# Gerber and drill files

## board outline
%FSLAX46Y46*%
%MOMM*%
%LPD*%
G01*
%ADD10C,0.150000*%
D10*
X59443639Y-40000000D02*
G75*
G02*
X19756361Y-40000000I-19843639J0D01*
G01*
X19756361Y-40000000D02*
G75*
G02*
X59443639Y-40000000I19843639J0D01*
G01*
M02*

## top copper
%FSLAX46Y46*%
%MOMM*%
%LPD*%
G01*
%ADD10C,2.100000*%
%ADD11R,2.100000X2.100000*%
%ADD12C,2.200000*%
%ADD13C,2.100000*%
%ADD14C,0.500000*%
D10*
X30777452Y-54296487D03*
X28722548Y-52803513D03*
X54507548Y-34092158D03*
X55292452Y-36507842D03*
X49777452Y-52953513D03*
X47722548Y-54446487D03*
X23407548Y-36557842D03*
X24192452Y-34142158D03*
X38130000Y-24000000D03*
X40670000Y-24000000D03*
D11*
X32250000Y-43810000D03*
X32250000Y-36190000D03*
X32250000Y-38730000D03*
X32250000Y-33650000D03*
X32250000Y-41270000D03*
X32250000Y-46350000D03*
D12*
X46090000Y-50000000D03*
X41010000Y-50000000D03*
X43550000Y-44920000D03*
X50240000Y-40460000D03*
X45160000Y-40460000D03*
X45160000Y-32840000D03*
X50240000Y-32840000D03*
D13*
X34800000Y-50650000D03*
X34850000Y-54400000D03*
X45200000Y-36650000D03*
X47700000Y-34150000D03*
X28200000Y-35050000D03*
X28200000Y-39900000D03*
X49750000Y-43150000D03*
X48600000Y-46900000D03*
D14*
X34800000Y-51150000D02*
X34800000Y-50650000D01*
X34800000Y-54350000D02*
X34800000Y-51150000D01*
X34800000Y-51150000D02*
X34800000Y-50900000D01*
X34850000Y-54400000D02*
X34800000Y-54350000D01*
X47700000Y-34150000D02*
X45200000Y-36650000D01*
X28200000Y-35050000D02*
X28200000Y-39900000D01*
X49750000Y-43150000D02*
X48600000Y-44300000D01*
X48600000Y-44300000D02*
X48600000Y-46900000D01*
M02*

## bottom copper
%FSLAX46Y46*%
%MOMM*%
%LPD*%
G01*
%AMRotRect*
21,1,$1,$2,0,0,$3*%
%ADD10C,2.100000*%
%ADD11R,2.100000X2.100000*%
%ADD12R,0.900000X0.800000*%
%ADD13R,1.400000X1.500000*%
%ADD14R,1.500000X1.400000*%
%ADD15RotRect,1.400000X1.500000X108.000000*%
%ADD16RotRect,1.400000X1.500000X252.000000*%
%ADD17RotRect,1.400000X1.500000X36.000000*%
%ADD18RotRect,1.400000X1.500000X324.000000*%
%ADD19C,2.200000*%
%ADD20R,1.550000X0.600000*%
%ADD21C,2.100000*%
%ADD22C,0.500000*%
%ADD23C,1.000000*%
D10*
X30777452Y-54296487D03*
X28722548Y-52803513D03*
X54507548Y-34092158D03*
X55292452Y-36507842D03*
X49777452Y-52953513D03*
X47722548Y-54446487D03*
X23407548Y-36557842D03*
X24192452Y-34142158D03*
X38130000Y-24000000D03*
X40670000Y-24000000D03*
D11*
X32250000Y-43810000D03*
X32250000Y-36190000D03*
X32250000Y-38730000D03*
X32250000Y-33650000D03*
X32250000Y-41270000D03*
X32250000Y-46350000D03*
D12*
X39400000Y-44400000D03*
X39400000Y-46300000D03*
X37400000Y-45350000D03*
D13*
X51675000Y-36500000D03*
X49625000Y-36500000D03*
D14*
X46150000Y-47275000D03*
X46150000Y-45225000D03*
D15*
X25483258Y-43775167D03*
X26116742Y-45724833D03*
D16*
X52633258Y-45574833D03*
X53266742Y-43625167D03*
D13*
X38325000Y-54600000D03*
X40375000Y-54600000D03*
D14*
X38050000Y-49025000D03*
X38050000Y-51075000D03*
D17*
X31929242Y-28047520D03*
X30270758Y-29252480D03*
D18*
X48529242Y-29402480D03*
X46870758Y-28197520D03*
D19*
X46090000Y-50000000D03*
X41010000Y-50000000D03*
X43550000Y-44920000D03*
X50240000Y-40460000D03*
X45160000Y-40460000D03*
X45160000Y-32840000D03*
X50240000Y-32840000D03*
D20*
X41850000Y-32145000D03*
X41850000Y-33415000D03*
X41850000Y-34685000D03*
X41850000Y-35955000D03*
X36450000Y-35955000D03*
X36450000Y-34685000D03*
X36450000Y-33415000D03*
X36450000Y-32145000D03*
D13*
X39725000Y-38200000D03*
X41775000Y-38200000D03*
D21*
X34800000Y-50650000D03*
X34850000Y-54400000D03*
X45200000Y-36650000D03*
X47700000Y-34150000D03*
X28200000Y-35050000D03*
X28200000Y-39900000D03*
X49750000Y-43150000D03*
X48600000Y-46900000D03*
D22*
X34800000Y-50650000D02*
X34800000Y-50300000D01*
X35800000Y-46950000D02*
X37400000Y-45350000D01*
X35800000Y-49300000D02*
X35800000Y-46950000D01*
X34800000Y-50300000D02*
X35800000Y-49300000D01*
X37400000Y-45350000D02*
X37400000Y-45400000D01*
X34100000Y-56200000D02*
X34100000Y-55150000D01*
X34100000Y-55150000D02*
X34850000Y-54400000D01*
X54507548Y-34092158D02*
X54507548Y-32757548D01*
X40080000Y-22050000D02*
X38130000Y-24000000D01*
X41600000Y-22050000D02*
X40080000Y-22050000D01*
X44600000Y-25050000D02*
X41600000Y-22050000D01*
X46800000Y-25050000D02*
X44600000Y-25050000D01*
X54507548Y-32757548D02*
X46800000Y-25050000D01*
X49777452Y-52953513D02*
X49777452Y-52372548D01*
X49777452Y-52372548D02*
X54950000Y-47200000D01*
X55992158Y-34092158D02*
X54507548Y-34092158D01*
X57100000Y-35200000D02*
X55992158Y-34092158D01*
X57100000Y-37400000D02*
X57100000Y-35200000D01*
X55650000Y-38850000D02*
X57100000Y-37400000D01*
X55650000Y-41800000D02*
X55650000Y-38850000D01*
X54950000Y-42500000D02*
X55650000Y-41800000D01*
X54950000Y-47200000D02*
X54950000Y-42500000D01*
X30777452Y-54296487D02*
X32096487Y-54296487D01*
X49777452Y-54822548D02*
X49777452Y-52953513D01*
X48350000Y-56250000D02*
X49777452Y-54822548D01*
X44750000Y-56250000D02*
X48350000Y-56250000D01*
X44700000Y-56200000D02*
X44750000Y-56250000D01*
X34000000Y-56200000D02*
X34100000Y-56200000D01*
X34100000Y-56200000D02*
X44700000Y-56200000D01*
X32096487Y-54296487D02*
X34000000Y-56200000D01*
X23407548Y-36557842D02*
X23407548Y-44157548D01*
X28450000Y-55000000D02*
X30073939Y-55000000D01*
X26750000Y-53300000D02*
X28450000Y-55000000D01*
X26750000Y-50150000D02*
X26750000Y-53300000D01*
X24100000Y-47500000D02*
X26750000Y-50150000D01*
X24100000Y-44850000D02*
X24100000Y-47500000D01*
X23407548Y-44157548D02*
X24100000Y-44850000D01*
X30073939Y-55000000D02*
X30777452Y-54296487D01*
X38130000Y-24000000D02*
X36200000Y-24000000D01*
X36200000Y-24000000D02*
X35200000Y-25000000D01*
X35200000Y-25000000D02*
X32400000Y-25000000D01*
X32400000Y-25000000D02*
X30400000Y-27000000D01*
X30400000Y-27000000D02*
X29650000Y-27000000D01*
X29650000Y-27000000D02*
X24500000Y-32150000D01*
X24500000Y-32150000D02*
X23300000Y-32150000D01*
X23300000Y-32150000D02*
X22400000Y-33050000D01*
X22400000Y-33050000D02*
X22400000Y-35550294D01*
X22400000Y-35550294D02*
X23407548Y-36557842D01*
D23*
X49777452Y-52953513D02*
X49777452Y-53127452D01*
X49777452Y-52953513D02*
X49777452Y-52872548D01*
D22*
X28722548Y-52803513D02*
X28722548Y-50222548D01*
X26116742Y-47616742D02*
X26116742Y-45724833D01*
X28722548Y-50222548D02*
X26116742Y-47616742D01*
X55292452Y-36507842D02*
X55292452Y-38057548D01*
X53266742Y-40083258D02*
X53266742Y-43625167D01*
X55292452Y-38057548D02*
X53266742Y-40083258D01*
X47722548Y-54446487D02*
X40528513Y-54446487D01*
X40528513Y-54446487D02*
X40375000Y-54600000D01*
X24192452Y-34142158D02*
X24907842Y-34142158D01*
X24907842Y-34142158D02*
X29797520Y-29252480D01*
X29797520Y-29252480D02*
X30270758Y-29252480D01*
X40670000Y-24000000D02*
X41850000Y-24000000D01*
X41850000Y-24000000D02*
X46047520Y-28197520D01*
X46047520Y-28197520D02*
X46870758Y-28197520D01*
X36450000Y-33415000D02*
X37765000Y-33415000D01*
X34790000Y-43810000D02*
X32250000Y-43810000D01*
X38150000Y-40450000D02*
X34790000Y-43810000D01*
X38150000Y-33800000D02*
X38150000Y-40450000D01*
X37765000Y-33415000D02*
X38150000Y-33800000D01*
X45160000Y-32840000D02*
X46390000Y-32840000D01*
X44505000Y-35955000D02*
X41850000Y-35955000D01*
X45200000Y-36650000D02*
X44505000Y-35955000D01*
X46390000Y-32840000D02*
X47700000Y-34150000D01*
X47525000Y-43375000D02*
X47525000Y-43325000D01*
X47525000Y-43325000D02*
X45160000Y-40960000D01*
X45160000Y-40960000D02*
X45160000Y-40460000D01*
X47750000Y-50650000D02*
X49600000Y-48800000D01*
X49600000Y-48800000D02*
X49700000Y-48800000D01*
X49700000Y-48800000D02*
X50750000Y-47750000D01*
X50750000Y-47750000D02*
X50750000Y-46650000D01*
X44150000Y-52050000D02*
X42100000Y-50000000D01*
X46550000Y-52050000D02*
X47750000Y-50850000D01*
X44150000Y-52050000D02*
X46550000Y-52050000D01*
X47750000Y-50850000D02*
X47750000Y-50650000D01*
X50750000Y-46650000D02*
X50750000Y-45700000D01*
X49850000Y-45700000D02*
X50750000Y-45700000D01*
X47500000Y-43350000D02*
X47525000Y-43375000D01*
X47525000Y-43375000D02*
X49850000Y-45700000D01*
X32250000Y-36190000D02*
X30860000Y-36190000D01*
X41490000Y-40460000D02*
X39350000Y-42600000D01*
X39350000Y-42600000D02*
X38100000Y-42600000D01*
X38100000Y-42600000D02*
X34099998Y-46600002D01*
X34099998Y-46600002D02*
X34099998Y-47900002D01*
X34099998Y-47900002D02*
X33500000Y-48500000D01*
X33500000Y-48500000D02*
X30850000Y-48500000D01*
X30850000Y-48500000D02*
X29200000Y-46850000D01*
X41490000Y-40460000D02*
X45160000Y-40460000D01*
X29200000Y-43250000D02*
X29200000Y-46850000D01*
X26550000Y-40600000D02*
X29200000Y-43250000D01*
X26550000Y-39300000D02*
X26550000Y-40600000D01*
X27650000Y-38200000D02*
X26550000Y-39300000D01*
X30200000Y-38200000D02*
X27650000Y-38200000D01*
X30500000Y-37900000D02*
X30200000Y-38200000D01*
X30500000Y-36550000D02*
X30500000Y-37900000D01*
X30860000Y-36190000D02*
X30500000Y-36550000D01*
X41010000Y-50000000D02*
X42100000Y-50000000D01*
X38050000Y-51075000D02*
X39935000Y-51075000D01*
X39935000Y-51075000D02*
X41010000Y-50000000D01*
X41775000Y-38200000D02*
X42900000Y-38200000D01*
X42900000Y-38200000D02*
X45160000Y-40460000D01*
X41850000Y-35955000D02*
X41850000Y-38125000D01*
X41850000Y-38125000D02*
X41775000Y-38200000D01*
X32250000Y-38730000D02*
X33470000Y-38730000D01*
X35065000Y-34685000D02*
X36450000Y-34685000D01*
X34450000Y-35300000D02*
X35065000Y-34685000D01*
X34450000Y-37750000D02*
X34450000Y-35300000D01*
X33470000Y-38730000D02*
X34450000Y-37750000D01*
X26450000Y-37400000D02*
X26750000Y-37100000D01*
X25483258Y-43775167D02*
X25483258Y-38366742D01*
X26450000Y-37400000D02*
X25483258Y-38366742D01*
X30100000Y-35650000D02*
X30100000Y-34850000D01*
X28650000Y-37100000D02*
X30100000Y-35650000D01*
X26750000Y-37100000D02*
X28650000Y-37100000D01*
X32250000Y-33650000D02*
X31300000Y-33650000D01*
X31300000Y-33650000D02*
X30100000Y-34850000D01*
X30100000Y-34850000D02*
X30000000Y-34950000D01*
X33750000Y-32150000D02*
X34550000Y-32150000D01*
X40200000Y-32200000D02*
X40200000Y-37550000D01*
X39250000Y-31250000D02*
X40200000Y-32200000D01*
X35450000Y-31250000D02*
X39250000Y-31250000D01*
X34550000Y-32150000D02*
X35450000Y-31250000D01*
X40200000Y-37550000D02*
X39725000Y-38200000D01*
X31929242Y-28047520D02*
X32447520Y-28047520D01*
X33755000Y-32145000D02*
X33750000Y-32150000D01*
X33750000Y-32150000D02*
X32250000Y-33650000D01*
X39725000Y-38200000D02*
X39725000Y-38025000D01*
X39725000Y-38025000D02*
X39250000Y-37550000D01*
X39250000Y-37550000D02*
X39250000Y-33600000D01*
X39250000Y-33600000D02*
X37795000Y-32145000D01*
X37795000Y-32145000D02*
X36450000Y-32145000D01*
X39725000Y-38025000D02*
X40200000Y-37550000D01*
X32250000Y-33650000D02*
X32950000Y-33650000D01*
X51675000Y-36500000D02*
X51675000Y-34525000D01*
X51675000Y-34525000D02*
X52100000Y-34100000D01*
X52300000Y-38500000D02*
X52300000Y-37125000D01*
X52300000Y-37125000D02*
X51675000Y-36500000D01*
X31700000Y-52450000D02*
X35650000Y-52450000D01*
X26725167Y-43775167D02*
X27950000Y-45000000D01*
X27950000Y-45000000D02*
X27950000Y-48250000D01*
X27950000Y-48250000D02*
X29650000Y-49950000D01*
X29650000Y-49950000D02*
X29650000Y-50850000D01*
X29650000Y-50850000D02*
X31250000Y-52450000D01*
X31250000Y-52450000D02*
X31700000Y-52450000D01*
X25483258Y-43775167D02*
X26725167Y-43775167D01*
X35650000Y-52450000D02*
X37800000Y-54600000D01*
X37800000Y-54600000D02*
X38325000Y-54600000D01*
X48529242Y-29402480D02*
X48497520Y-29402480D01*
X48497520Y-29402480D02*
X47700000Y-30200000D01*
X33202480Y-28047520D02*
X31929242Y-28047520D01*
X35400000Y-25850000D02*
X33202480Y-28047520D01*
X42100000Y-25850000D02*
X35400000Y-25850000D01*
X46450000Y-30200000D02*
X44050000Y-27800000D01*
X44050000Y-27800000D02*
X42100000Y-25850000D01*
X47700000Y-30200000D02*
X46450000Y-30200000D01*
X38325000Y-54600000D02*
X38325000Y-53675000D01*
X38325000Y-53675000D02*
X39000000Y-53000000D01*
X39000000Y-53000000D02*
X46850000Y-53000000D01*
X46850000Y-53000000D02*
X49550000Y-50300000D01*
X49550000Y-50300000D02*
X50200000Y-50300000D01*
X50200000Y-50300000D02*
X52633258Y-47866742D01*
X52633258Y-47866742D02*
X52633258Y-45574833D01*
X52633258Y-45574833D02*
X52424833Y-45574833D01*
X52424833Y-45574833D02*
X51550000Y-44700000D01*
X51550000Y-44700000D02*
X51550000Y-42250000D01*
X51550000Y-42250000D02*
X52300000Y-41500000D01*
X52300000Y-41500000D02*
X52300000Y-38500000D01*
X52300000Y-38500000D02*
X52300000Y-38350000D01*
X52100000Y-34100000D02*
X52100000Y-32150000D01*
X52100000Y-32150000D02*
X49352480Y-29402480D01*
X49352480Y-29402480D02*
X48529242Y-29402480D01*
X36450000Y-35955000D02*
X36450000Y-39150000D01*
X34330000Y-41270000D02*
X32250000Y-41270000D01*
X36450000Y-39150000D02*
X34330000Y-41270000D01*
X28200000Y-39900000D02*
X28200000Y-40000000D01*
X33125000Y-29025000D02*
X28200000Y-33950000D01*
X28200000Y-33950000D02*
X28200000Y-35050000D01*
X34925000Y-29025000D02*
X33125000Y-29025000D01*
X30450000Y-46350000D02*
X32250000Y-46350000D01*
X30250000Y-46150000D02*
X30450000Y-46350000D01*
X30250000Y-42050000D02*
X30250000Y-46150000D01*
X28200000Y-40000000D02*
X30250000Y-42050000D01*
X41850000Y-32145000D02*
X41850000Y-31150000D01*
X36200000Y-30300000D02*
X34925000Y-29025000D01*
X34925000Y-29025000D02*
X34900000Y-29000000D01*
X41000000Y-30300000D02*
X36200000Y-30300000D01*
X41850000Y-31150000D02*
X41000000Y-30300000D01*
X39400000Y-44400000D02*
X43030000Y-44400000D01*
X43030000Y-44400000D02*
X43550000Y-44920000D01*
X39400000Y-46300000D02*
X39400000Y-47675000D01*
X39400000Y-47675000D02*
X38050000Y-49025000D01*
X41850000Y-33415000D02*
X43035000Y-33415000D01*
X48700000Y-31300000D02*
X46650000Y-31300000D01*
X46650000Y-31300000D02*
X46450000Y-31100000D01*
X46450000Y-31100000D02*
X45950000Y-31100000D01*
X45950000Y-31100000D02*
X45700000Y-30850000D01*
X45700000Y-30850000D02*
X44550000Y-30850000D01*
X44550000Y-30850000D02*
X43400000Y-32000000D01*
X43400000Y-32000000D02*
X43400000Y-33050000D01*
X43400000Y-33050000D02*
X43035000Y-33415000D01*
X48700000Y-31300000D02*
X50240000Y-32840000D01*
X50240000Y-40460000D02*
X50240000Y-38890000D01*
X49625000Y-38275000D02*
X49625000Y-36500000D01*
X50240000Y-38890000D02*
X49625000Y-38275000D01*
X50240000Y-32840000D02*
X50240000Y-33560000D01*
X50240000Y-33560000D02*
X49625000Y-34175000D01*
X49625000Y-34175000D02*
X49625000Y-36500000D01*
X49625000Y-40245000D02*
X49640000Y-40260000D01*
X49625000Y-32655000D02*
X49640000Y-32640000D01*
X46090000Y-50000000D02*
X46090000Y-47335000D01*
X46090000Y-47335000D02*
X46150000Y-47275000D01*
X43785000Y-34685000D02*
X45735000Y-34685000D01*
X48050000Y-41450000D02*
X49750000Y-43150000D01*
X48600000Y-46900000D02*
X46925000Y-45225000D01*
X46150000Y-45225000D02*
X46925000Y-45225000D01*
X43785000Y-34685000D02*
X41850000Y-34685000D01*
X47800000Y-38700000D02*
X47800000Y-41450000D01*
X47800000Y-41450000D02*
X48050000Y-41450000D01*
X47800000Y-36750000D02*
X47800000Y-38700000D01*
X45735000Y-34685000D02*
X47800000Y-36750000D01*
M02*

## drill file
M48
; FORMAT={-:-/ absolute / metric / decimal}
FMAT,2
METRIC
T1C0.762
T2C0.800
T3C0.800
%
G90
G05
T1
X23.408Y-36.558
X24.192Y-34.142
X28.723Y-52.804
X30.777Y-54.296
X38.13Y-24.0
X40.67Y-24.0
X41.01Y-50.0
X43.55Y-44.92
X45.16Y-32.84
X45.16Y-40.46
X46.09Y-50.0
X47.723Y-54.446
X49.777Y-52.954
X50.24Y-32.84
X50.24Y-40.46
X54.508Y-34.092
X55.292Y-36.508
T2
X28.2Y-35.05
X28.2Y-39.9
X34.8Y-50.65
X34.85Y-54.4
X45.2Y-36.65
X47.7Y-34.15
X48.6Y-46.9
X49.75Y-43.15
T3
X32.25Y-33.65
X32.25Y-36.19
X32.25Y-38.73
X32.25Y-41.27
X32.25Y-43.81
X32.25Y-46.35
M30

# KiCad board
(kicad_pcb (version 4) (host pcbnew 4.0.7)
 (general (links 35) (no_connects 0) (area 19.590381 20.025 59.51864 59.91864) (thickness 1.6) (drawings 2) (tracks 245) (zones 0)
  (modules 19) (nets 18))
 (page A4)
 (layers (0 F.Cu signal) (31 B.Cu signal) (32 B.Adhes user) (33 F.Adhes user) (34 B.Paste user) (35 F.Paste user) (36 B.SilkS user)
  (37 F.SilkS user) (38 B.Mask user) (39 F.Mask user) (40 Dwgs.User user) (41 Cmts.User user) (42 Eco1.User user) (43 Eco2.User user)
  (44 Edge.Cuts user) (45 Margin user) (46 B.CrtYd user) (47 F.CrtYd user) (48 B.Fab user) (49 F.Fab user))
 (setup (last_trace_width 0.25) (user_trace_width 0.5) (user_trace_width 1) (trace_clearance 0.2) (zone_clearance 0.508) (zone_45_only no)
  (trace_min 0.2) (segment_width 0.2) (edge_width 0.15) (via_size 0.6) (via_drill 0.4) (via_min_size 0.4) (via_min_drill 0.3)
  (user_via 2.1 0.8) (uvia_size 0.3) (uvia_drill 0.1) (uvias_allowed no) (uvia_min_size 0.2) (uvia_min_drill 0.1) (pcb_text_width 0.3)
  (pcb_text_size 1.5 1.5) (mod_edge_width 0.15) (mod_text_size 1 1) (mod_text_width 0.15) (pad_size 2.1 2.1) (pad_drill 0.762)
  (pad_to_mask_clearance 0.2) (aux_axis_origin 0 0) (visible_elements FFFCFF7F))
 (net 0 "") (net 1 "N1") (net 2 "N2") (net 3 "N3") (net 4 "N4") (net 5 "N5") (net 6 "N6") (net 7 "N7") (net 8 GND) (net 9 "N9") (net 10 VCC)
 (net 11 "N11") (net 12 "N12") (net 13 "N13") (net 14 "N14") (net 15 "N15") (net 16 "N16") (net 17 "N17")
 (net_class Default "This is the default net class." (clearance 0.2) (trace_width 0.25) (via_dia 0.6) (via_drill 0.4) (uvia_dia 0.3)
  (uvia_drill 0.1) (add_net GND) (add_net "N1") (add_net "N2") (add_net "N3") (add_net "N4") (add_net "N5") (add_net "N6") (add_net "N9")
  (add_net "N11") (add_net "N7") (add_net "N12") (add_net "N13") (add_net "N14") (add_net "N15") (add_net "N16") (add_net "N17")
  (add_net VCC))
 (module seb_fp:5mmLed (layer F.Cu) (at 29.75 53.55 144)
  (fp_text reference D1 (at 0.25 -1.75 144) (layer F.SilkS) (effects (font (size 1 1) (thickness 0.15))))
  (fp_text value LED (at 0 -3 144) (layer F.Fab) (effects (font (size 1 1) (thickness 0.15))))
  (pad 1 thru_hole circle (at -1.27 0 144) (size 2.1 2.1) (drill 0.762) (layers *.Cu *.Mask) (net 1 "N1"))
  (pad 2 thru_hole circle (at 1.27 0 144) (size 2.1 2.1) (drill 0.762) (layers *.Cu *.Mask) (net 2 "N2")))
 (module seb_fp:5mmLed (layer F.Cu) (at 54.9 35.3 288)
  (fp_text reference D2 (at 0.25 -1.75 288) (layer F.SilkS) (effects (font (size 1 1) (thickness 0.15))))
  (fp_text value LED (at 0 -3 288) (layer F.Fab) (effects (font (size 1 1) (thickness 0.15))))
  (pad 1 thru_hole circle (at -1.27 0 288) (size 2.1 2.1) (drill 0.762) (layers *.Cu *.Mask) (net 1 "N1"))
  (pad 2 thru_hole circle (at 1.27 0 288) (size 2.1 2.1) (drill 0.762) (layers *.Cu *.Mask) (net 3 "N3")))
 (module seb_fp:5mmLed (layer F.Cu) (at 48.75 53.7 216)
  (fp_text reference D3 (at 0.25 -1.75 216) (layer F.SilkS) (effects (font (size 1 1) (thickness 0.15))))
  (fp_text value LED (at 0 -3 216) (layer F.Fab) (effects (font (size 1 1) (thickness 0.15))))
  (pad 1 thru_hole circle (at -1.27 0 216) (size 2.1 2.1) (drill 0.762) (layers *.Cu *.Mask) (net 1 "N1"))
  (pad 2 thru_hole circle (at 1.27 0 216) (size 2.1 2.1) (drill 0.762) (layers *.Cu *.Mask) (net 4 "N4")))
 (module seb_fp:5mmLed (layer F.Cu) (at 23.8 35.35 72)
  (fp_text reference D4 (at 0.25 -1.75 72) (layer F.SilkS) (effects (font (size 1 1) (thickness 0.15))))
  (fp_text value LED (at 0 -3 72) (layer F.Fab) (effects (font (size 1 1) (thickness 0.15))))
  (pad 1 thru_hole circle (at -1.27 0 144) (size 2.1 2.1) (drill 0.762) (layers *.Cu *.Mask) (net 1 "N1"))
  (pad 2 thru_hole circle (at 1.27 0 144) (size 2.1 2.1) (drill 0.762) (layers *.Cu *.Mask) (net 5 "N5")))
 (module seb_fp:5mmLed (layer F.Cu) (at 39.4 24)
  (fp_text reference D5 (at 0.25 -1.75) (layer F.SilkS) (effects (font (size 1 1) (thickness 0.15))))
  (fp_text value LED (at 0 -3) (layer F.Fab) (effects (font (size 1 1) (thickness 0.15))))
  (pad 1 thru_hole circle (at -1.27 0) (size 2.1 2.1) (drill 0.762) (layers *.Cu *.Mask) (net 1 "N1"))
  (pad 2 thru_hole circle (at 1.27 0) (size 2.1 2.1) (drill 0.762) (layers *.Cu *.Mask) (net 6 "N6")))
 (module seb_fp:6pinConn (layer F.Cu) (at 32.25 40)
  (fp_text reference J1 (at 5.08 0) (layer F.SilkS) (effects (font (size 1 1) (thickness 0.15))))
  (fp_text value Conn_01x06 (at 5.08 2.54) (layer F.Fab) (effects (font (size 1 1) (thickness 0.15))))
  (pad 5 thru_hole rect (at 0 3.81) (size 2.1 2.1) (drill 0.8) (layers *.Cu *.Mask) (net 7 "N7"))
  (pad 2 thru_hole rect (at 0 -3.81) (size 2.1 2.1) (drill 0.8) (layers *.Cu *.Mask) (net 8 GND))
  (pad 3 thru_hole rect (at 0 -1.27) (size 2.1 2.1) (drill 0.8) (layers *.Cu *.Mask) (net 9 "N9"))
  (pad 1 thru_hole rect (at 0 -6.35) (size 2.1 2.1) (drill 0.8) (layers *.Cu *.Mask) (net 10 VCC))
  (pad 4 thru_hole rect (at 0 1.27) (size 2.1 2.1) (drill 0.8) (layers *.Cu *.Mask) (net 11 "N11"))
  (pad 6 thru_hole rect (at 0 6.35) (size 2.1 2.1) (drill 0.8) (layers *.Cu *.Mask) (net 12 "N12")))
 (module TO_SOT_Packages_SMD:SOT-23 (layer B.Cu) (at 38.4 45.35 180)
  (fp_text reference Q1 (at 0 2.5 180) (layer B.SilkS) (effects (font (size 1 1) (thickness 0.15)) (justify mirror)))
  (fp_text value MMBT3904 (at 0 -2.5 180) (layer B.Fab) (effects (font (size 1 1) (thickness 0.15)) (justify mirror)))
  (pad 1 smd rect (at -1 0.95 180) (size 0.9 0.8) (layers B.Cu B.Paste B.Mask) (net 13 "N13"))
  (pad 2 smd rect (at -1 -0.95 180) (size 0.9 0.8) (layers B.Cu B.Paste B.Mask) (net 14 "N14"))
  (pad 3 smd rect (at 1 0 180) (size 0.9 0.8) (layers B.Cu B.Paste B.Mask) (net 1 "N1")))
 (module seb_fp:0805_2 (layer B.Cu) (at 50.65 36.5)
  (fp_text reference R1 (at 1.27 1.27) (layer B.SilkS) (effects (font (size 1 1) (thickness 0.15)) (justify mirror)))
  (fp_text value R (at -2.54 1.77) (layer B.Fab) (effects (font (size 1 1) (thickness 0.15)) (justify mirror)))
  (pad 1 smd rect (at 1.025 0) (size 1.4 1.5) (layers B.Cu B.Paste B.Mask) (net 10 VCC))
  (pad 2 smd rect (at -1.025 0) (size 1.4 1.5) (layers B.Cu B.Paste B.Mask) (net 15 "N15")))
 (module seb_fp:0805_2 (layer B.Cu) (at 46.15 46.25 270)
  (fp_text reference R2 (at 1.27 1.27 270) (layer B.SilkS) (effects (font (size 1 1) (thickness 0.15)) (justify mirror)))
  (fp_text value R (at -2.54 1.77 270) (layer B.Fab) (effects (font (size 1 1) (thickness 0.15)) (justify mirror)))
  (pad 1 smd rect (at 1.025 0 270) (size 1.4 1.5) (layers B.Cu B.Paste B.Mask) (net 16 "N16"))
  (pad 2 smd rect (at -1.025 0 270) (size 1.4 1.5) (layers B.Cu B.Paste B.Mask) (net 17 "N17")))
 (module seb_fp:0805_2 (layer B.Cu) (at 25.8 44.75 108)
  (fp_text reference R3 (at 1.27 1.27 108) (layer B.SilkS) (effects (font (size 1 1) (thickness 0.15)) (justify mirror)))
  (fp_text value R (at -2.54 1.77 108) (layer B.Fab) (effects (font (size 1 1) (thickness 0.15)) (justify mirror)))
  (pad 1 smd rect (at 1.025 0 108) (size 1.4 1.5) (layers B.Cu B.Paste B.Mask) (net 10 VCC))
  (pad 2 smd rect (at -1.025 0 108) (size 1.4 1.5) (layers B.Cu B.Paste B.Mask) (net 2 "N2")))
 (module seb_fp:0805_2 (layer B.Cu) (at 52.95 44.6 252)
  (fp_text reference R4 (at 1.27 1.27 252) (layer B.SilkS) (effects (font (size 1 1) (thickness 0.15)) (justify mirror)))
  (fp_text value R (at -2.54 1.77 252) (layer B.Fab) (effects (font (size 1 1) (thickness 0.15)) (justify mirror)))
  (pad 1 smd rect (at 1.025 0 252) (size 1.4 1.5) (layers B.Cu B.Paste B.Mask) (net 10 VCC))
  (pad 2 smd rect (at -1.025 0 252) (size 1.4 1.5) (layers B.Cu B.Paste B.Mask) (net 3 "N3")))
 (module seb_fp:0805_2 (layer B.Cu) (at 39.35 54.6 180)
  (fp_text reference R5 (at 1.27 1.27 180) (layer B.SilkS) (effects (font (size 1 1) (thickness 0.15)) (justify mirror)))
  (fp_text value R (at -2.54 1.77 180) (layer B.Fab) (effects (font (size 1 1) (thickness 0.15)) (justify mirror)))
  (pad 1 smd rect (at 1.025 0 180) (size 1.4 1.5) (layers B.Cu B.Paste B.Mask) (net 10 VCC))
  (pad 2 smd rect (at -1.025 0 180) (size 1.4 1.5) (layers B.Cu B.Paste B.Mask) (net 4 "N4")))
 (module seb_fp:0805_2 (layer B.Cu) (at 38.05 50.05 90)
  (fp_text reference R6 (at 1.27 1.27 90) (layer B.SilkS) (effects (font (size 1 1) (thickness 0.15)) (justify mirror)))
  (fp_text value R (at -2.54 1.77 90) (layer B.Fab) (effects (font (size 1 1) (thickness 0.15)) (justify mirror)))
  (pad 1 smd rect (at 1.025 0 90) (size 1.4 1.5) (layers B.Cu B.Paste B.Mask) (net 14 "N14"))
  (pad 2 smd rect (at -1.025 0 90) (size 1.4 1.5) (layers B.Cu B.Paste B.Mask) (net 8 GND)))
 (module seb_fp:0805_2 (layer B.Cu) (at 31.1 28.65 36)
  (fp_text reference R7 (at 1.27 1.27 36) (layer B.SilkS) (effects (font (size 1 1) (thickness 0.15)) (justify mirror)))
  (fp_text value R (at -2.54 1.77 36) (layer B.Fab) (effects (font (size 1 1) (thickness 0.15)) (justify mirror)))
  (pad 1 smd rect (at 1.025 0 36) (size 1.4 1.5) (layers B.Cu B.Paste B.Mask) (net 10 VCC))
  (pad 2 smd rect (at -1.025 0 36) (size 1.4 1.5) (layers B.Cu B.Paste B.Mask) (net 5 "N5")))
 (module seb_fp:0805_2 (layer B.Cu) (at 47.7 28.8 324)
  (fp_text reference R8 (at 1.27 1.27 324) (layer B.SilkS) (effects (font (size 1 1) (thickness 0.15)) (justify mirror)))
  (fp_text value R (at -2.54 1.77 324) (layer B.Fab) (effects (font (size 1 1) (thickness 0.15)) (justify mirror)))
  (pad 1 smd rect (at 1.025 0 324) (size 1.4 1.5) (layers B.Cu B.Paste B.Mask) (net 10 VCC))
  (pad 2 smd rect (at -1.025 0 324) (size 1.4 1.5) (layers B.Cu B.Paste B.Mask) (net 6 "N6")))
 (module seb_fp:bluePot (layer F.Cu) (at 43.55 50 180)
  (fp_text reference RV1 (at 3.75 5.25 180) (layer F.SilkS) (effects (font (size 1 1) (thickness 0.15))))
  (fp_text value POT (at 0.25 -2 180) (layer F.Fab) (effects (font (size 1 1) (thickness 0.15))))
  (pad 1 thru_hole circle (at -2.54 0 180) (size 2.2 2.2) (drill 0.762) (layers *.Cu *.Mask) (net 16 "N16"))
  (pad 3 thru_hole circle (at 2.54 0 180) (size 2.2 2.2) (drill 0.762) (layers *.Cu *.Mask) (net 8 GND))
  (pad 2 thru_hole circle (at 0 5.08 180) (size 2.2 2.2) (drill 0.762) (layers *.Cu *.Mask) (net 13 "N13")))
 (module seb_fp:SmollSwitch (layer F.Cu) (at 47.7 36.65 90)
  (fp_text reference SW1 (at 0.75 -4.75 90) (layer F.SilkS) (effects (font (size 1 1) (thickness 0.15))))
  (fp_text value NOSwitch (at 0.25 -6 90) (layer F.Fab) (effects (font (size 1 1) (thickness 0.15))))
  (pad 1 thru_hole circle (at -3.81 2.54 90) (size 2.2 2.2) (drill 0.762) (layers *.Cu *.Mask) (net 15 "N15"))
  (pad 2 thru_hole circle (at -3.81 -2.54 90) (size 2.2 2.2) (drill 0.762) (layers *.Cu *.Mask) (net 8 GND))
  (pad 2 thru_hole circle (at 3.81 -2.54 90) (size 2.2 2.2) (drill 0.762) (layers *.Cu *.Mask) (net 8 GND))
  (pad 1 thru_hole circle (at 3.81 2.54 90) (size 2.2 2.2) (drill 0.762) (layers *.Cu *.Mask) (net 15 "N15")))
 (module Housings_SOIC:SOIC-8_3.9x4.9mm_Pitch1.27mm (layer B.Cu) (at 39.15 34.05 180)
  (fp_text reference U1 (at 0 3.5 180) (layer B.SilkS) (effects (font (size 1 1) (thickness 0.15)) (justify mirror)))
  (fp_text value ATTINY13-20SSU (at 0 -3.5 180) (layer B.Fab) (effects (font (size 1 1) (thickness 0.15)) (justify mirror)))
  (pad 1 smd rect (at -2.7 1.905 180) (size 1.55 0.6) (layers B.Cu B.Paste B.Mask) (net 12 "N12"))
  (pad 2 smd rect (at -2.7 0.635 180) (size 1.55 0.6) (layers B.Cu B.Paste B.Mask) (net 15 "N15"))
  (pad 3 smd rect (at -2.7 -0.635 180) (size 1.55 0.6) (layers B.Cu B.Paste B.Mask) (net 17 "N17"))
  (pad 4 smd rect (at -2.7 -1.905 180) (size 1.55 0.6) (layers B.Cu B.Paste B.Mask) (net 8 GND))
  (pad 5 smd rect (at 2.7 -1.905 180) (size 1.55 0.6) (layers B.Cu B.Paste B.Mask) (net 11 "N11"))
  (pad 6 smd rect (at 2.7 -0.635 180) (size 1.55 0.6) (layers B.Cu B.Paste B.Mask) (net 9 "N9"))
  (pad 7 smd rect (at 2.7 0.635 180) (size 1.55 0.6) (layers B.Cu B.Paste B.Mask) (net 7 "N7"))
  (pad 8 smd rect (at 2.7 1.905 180) (size 1.55 0.6) (layers B.Cu B.Paste B.Mask) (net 10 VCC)))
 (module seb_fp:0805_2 (layer B.Cu) (at 40.75 38.2 180)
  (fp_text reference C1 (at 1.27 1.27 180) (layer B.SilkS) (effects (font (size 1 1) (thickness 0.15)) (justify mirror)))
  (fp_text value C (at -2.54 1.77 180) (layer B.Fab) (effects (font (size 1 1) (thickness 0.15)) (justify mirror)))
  (pad 1 smd rect (at 1.025 0 180) (size 1.4 1.5) (layers B.Cu B.Paste B.Mask) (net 10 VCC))
  (pad 2 smd rect (at -1.025 0 180) (size 1.4 1.5) (layers B.Cu B.Paste B.Mask) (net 8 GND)))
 (gr_circle (center 39.6 40) (end 56.5 50.4) (layer Edge.Cuts) (width 0.15))
 (segment (start 34.8 50.65) (end 34.8 50.3) (width 0.5) (layer B.Cu) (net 1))
 (via (at 34.8 50.65) (size 2.1) (drill 0.8) (layers F.Cu B.Cu) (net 1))
 (segment (start 34.8 51.15) (end 34.8 50.65) (width 0.5) (layer F.Cu) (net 1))
 (segment (start 35.8 46.95) (end 37.4 45.35) (width 0.5) (layer B.Cu) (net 1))
 (segment (start 35.8 49.3) (end 35.8 46.95) (width 0.5) (layer B.Cu) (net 1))
 (segment (start 34.8 50.3) (end 35.8 49.3) (width 0.5) (layer B.Cu) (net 1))
 (segment (start 37.4 45.35) (end 37.4 45.4) (width 0.5) (layer B.Cu) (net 1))
 (segment (start 34.1 56.2) (end 34.1 55.15) (width 0.5) (layer B.Cu) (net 1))
 (segment (start 34.8 54.35) (end 34.8 51.15) (width 0.5) (layer F.Cu) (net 1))
 (segment (start 34.8 51.15) (end 34.8 50.9) (width 0.5) (layer F.Cu) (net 1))
 (segment (start 34.85 54.4) (end 34.8 54.35) (width 0.5) (layer F.Cu) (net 1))
 (via (at 34.85 54.4) (size 2.1) (drill 0.8) (layers F.Cu B.Cu) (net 1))
 (segment (start 34.1 55.15) (end 34.85 54.4) (width 0.5) (layer B.Cu) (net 1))
 (segment (start 54.507548 34.092158) (end 54.507548 32.757548) (width 0.5) (layer B.Cu) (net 1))
 (segment (start 40.08 22.05) (end 38.13 24) (width 0.5) (layer B.Cu) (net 1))
 (segment (start 41.6 22.05) (end 40.08 22.05) (width 0.5) (layer B.Cu) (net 1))
 (segment (start 44.6 25.05) (end 41.6 22.05) (width 0.5) (layer B.Cu) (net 1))
 (segment (start 46.8 25.05) (end 44.6 25.05) (width 0.5) (layer B.Cu) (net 1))
 (segment (start 54.507548 32.757548) (end 46.8 25.05) (width 0.5) (layer B.Cu) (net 1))
 (segment (start 49.777452 52.953513) (end 49.777452 52.372548) (width 0.5) (layer B.Cu) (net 1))
 (segment (start 49.777452 52.372548) (end 54.95 47.2) (width 0.5) (layer B.Cu) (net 1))
 (segment (start 55.992158 34.092158) (end 54.507548 34.092158) (width 0.5) (layer B.Cu) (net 1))
 (segment (start 57.1 35.2) (end 55.992158 34.092158) (width 0.5) (layer B.Cu) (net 1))
 (segment (start 57.1 37.4) (end 57.1 35.2) (width 0.5) (layer B.Cu) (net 1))
 (segment (start 55.65 38.85) (end 57.1 37.4) (width 0.5) (layer B.Cu) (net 1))
 (segment (start 55.65 41.8) (end 55.65 38.85) (width 0.5) (layer B.Cu) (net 1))
 (segment (start 54.95 42.5) (end 55.65 41.8) (width 0.5) (layer B.Cu) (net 1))
 (segment (start 54.95 47.2) (end 54.95 42.5) (width 0.5) (layer B.Cu) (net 1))
 (segment (start 30.777452 54.296487) (end 32.096487 54.296487) (width 0.5) (layer B.Cu) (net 1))
 (segment (start 49.777452 54.822548) (end 49.777452 52.953513) (width 0.5) (layer B.Cu) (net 1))
 (segment (start 48.35 56.25) (end 49.777452 54.822548) (width 0.5) (layer B.Cu) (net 1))
 (segment (start 44.75 56.25) (end 48.35 56.25) (width 0.5) (layer B.Cu) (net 1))
 (segment (start 44.7 56.2) (end 44.75 56.25) (width 0.5) (layer B.Cu) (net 1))
 (segment (start 34 56.2) (end 34.1 56.2) (width 0.5) (layer B.Cu) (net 1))
 (segment (start 34.1 56.2) (end 44.7 56.2) (width 0.5) (layer B.Cu) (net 1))
 (segment (start 32.096487 54.296487) (end 34 56.2) (width 0.5) (layer B.Cu) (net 1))
 (segment (start 23.407548 36.557842) (end 23.407548 44.157548) (width 0.5) (layer B.Cu) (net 1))
 (segment (start 28.45 55) (end 30.073939 55) (width 0.5) (layer B.Cu) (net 1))
 (segment (start 26.75 53.3) (end 28.45 55) (width 0.5) (layer B.Cu) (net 1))
 (segment (start 26.75 50.15) (end 26.75 53.3) (width 0.5) (layer B.Cu) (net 1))
 (segment (start 24.1 47.5) (end 26.75 50.15) (width 0.5) (layer B.Cu) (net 1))
 (segment (start 24.1 44.85) (end 24.1 47.5) (width 0.5) (layer B.Cu) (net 1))
 (segment (start 23.407548 44.157548) (end 24.1 44.85) (width 0.5) (layer B.Cu) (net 1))
 (segment (start 30.073939 55) (end 30.777452 54.296487) (width 0.5) (layer B.Cu) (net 1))
 (segment (start 38.13 24) (end 36.2 24) (width 0.5) (layer B.Cu) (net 1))
 (segment (start 36.2 24) (end 35.2 25) (width 0.5) (layer B.Cu) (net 1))
 (segment (start 35.2 25) (end 32.4 25) (width 0.5) (layer B.Cu) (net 1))
 (segment (start 32.4 25) (end 30.4 27) (width 0.5) (layer B.Cu) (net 1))
 (segment (start 30.4 27) (end 29.65 27) (width 0.5) (layer B.Cu) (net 1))
 (segment (start 29.65 27) (end 24.5 32.15) (width 0.5) (layer B.Cu) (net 1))
 (segment (start 24.5 32.15) (end 23.3 32.15) (width 0.5) (layer B.Cu) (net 1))
 (segment (start 23.3 32.15) (end 22.4 33.05) (width 0.5) (layer B.Cu) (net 1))
 (segment (start 22.4 33.05) (end 22.4 35.550294) (width 0.5) (layer B.Cu) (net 1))
 (segment (start 22.4 35.550294) (end 23.407548 36.557842) (width 0.5) (layer B.Cu) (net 1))
 (segment (start 49.777452 52.953513) (end 49.777452 53.127452) (width 1) (layer B.Cu) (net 1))
 (segment (start 49.777452 52.953513) (end 49.777452 52.872548) (width 1) (layer B.Cu) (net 1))
 (segment (start 28.722548 52.803513) (end 28.722548 50.222548) (width 0.5) (layer B.Cu) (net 2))
 (segment (start 26.116742 47.616742) (end 26.116742 45.724833) (width 0.5) (layer B.Cu) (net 2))
 (segment (start 28.722548 50.222548) (end 26.116742 47.616742) (width 0.5) (layer B.Cu) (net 2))
 (segment (start 55.292452 36.507842) (end 55.292452 38.057548) (width 0.5) (layer B.Cu) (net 3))
 (segment (start 53.266742 40.083258) (end 53.266742 43.625167) (width 0.5) (layer B.Cu) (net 3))
 (segment (start 55.292452 38.057548) (end 53.266742 40.083258) (width 0.5) (layer B.Cu) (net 3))
 (segment (start 47.722548 54.446487) (end 40.528513 54.446487) (width 0.5) (layer B.Cu) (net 4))
 (segment (start 40.528513 54.446487) (end 40.375 54.6) (width 0.5) (layer B.Cu) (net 4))
 (segment (start 24.192452 34.142158) (end 24.907842 34.142158) (width 0.5) (layer B.Cu) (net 5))
 (segment (start 24.907842 34.142158) (end 29.79752 29.25248) (width 0.5) (layer B.Cu) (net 5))
 (segment (start 29.79752 29.25248) (end 30.270758 29.25248) (width 0.5) (layer B.Cu) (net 5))
 (segment (start 40.67 24) (end 41.85 24) (width 0.5) (layer B.Cu) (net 6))
 (segment (start 41.85 24) (end 46.04752 28.19752) (width 0.5) (layer B.Cu) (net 6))
 (segment (start 46.04752 28.19752) (end 46.870758 28.19752) (width 0.5) (layer B.Cu) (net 6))
 (segment (start 36.45 33.415) (end 37.765 33.415) (width 0.5) (layer B.Cu) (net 7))
 (segment (start 34.79 43.81) (end 32.25 43.81) (width 0.5) (layer B.Cu) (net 7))
 (segment (start 38.15 40.45) (end 34.79 43.81) (width 0.5) (layer B.Cu) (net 7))
 (segment (start 38.15 33.8) (end 38.15 40.45) (width 0.5) (layer B.Cu) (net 7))
 (segment (start 37.765 33.415) (end 38.15 33.8) (width 0.5) (layer B.Cu) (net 7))
 (segment (start 45.16 32.84) (end 46.39 32.84) (width 0.5) (layer B.Cu) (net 8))
 (segment (start 44.505 35.955) (end 41.85 35.955) (width 0.5) (layer B.Cu) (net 8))
 (segment (start 45.2 36.65) (end 44.505 35.955) (width 0.5) (layer B.Cu) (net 8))
 (via (at 45.2 36.65) (size 2.1) (drill 0.8) (layers F.Cu B.Cu) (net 8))
 (segment (start 47.7 34.15) (end 45.2 36.65) (width 0.5) (layer F.Cu) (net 8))
 (via (at 47.7 34.15) (size 2.1) (drill 0.8) (layers F.Cu B.Cu) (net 8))
 (segment (start 46.39 32.84) (end 47.7 34.15) (width 0.5) (layer B.Cu) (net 8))
 (segment (start 47.525 43.375) (end 47.525 43.325) (width 0.5) (layer B.Cu) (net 8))
 (segment (start 47.525 43.325) (end 45.16 40.96) (width 0.5) (layer B.Cu) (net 8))
 (segment (start 45.16 40.96) (end 45.16 40.46) (width 0.5) (layer B.Cu) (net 8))
 (segment (start 47.75 50.65) (end 49.6 48.8) (width 0.5) (layer B.Cu) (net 8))
 (segment (start 49.6 48.8) (end 49.7 48.8) (width 0.5) (layer B.Cu) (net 8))
 (segment (start 49.7 48.8) (end 50.75 47.75) (width 0.5) (layer B.Cu) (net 8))
 (segment (start 50.75 47.75) (end 50.75 46.65) (width 0.5) (layer B.Cu) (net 8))
 (segment (start 44.15 52.05) (end 42.1 50) (width 0.5) (layer B.Cu) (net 8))
 (segment (start 46.55 52.05) (end 47.75 50.85) (width 0.5) (layer B.Cu) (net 8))
 (segment (start 44.15 52.05) (end 46.55 52.05) (width 0.5) (layer B.Cu) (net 8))
 (segment (start 47.75 50.85) (end 47.75 50.65) (width 0.5) (layer B.Cu) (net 8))
 (segment (start 50.75 46.65) (end 50.75 45.7) (width 0.5) (layer B.Cu) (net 8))
 (segment (start 49.85 45.7) (end 50.75 45.7) (width 0.5) (layer B.Cu) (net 8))
 (segment (start 47.5 43.35) (end 47.525 43.375) (width 0.5) (layer B.Cu) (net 8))
 (segment (start 47.525 43.375) (end 49.85 45.7) (width 0.5) (layer B.Cu) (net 8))
 (segment (start 32.25 36.19) (end 30.86 36.19) (width 0.5) (layer B.Cu) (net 8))
 (segment (start 41.49 40.46) (end 39.35 42.6) (width 0.5) (layer B.Cu) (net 8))
 (segment (start 39.35 42.6) (end 38.1 42.6) (width 0.5) (layer B.Cu) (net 8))
 (segment (start 38.1 42.6) (end 34.099998 46.600002) (width 0.5) (layer B.Cu) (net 8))
 (segment (start 34.099998 46.600002) (end 34.099998 47.900002) (width 0.5) (layer B.Cu) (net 8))
 (segment (start 34.099998 47.900002) (end 33.5 48.5) (width 0.5) (layer B.Cu) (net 8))
 (segment (start 33.5 48.5) (end 30.85 48.5) (width 0.5) (layer B.Cu) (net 8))
 (segment (start 30.85 48.5) (end 29.2 46.85) (width 0.5) (layer B.Cu) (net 8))
 (segment (start 41.49 40.46) (end 45.16 40.46) (width 0.5) (layer B.Cu) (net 8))
 (segment (start 29.2 43.25) (end 29.2 46.85) (width 0.5) (layer B.Cu) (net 8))
 (segment (start 26.55 40.6) (end 29.2 43.25) (width 0.5) (layer B.Cu) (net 8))
 (segment (start 26.55 39.3) (end 26.55 40.6) (width 0.5) (layer B.Cu) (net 8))
 (segment (start 27.65 38.2) (end 26.55 39.3) (width 0.5) (layer B.Cu) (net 8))
 (segment (start 30.2 38.2) (end 27.65 38.2) (width 0.5) (layer B.Cu) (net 8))
 (segment (start 30.5 37.9) (end 30.2 38.2) (width 0.5) (layer B.Cu) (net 8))
 (segment (start 30.5 36.55) (end 30.5 37.9) (width 0.5) (layer B.Cu) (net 8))
 (segment (start 30.86 36.19) (end 30.5 36.55) (width 0.5) (layer B.Cu) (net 8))
 (segment (start 41.01 50) (end 42.1 50) (width 0.5) (layer B.Cu) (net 8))
 (segment (start 38.05 51.075) (end 39.935 51.075) (width 0.5) (layer B.Cu) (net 8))
 (segment (start 39.935 51.075) (end 41.01 50) (width 0.5) (layer B.Cu) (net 8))
 (segment (start 41.775 38.2) (end 42.9 38.2) (width 0.5) (layer B.Cu) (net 8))
 (segment (start 42.9 38.2) (end 45.16 40.46) (width 0.5) (layer B.Cu) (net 8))
 (segment (start 41.85 35.955) (end 41.85 38.125) (width 0.5) (layer B.Cu) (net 8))
 (segment (start 41.85 38.125) (end 41.775 38.2) (width 0.5) (layer B.Cu) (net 8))
 (segment (start 32.25 38.73) (end 33.47 38.73) (width 0.5) (layer B.Cu) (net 9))
 (segment (start 35.065 34.685) (end 36.45 34.685) (width 0.5) (layer B.Cu) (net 9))
 (segment (start 34.45 35.3) (end 35.065 34.685) (width 0.5) (layer B.Cu) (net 9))
 (segment (start 34.45 37.75) (end 34.45 35.3) (width 0.5) (layer B.Cu) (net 9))
 (segment (start 33.47 38.73) (end 34.45 37.75) (width 0.5) (layer B.Cu) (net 9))
 (segment (start 26.45 37.4) (end 26.75 37.1) (width 0.5) (layer B.Cu) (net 10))
 (segment (start 25.483258 43.775167) (end 25.483258 38.366742) (width 0.5) (layer B.Cu) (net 10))
 (segment (start 26.45 37.4) (end 25.483258 38.366742) (width 0.5) (layer B.Cu) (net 10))
 (segment (start 30.1 35.65) (end 30.1 34.85) (width 0.5) (layer B.Cu) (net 10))
 (segment (start 28.65 37.1) (end 30.1 35.65) (width 0.5) (layer B.Cu) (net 10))
 (segment (start 26.75 37.1) (end 28.65 37.1) (width 0.5) (layer B.Cu) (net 10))
 (segment (start 32.25 33.65) (end 31.3 33.65) (width 0.5) (layer B.Cu) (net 10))
 (segment (start 31.3 33.65) (end 30.1 34.85) (width 0.5) (layer B.Cu) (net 10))
 (segment (start 30.1 34.85) (end 30 34.95) (width 0.5) (layer B.Cu) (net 10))
 (segment (start 33.75 32.15) (end 34.55 32.15) (width 0.5) (layer B.Cu) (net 10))
 (segment (start 40.2 32.2) (end 40.2 37.55) (width 0.5) (layer B.Cu) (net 10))
 (segment (start 39.25 31.25) (end 40.2 32.2) (width 0.5) (layer B.Cu) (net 10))
 (segment (start 35.45 31.25) (end 39.25 31.25) (width 0.5) (layer B.Cu) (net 10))
 (segment (start 34.55 32.15) (end 35.45 31.25) (width 0.5) (layer B.Cu) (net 10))
 (segment (start 40.2 37.55) (end 39.725 38.2) (width 0.5) (layer B.Cu) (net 10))
 (segment (start 31.929242 28.04752) (end 32.44752 28.04752) (width 0.5) (layer B.Cu) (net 10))
 (segment (start 33.755 32.145) (end 33.75 32.15) (width 0.5) (layer B.Cu) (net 10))
 (segment (start 33.75 32.15) (end 32.25 33.65) (width 0.5) (layer B.Cu) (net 10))
 (segment (start 39.725 38.2) (end 39.725 38.025) (width 0.5) (layer B.Cu) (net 10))
 (segment (start 39.725 38.025) (end 39.25 37.55) (width 0.5) (layer B.Cu) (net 10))
 (segment (start 39.25 37.55) (end 39.25 33.6) (width 0.5) (layer B.Cu) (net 10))
 (segment (start 39.25 33.6) (end 37.795 32.145) (width 0.5) (layer B.Cu) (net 10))
 (segment (start 37.795 32.145) (end 36.45 32.145) (width 0.5) (layer B.Cu) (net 10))
 (segment (start 39.725 38.025) (end 40.2 37.55) (width 0.5) (layer B.Cu) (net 10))
 (segment (start 32.25 33.65) (end 32.95 33.65) (width 0.5) (layer B.Cu) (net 10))
 (segment (start 51.675 36.5) (end 51.675 34.525) (width 0.5) (layer B.Cu) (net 10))
 (segment (start 51.675 34.525) (end 52.1 34.1) (width 0.5) (layer B.Cu) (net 10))
 (segment (start 52.3 38.5) (end 52.3 37.125) (width 0.5) (layer B.Cu) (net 10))
 (segment (start 52.3 37.125) (end 51.675 36.5) (width 0.5) (layer B.Cu) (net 10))
 (segment (start 31.7 52.45) (end 35.65 52.45) (width 0.5) (layer B.Cu) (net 10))
 (segment (start 26.725167 43.775167) (end 27.95 45) (width 0.5) (layer B.Cu) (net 10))
 (segment (start 27.95 45) (end 27.95 48.25) (width 0.5) (layer B.Cu) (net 10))
 (segment (start 27.95 48.25) (end 29.65 49.95) (width 0.5) (layer B.Cu) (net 10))
 (segment (start 29.65 49.95) (end 29.65 50.85) (width 0.5) (layer B.Cu) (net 10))
 (segment (start 29.65 50.85) (end 31.25 52.45) (width 0.5) (layer B.Cu) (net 10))
 (segment (start 31.25 52.45) (end 31.7 52.45) (width 0.5) (layer B.Cu) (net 10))
 (segment (start 25.483258 43.775167) (end 26.725167 43.775167) (width 0.5) (layer B.Cu) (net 10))
 (segment (start 35.65 52.45) (end 37.8 54.6) (width 0.5) (layer B.Cu) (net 10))
 (segment (start 37.8 54.6) (end 38.325 54.6) (width 0.5) (layer B.Cu) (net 10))
 (segment (start 48.529242 29.40248) (end 48.49752 29.40248) (width 0.5) (layer B.Cu) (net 10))
 (segment (start 48.49752 29.40248) (end 47.7 30.2) (width 0.5) (layer B.Cu) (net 10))
 (segment (start 33.20248 28.04752) (end 31.929242 28.04752) (width 0.5) (layer B.Cu) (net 10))
 (segment (start 35.4 25.85) (end 33.20248 28.04752) (width 0.5) (layer B.Cu) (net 10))
 (segment (start 42.1 25.85) (end 35.4 25.85) (width 0.5) (layer B.Cu) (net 10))
 (segment (start 46.45 30.2) (end 44.05 27.8) (width 0.5) (layer B.Cu) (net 10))
 (segment (start 44.05 27.8) (end 42.1 25.85) (width 0.5) (layer B.Cu) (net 10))
 (segment (start 47.7 30.2) (end 46.45 30.2) (width 0.5) (layer B.Cu) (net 10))
 (segment (start 38.325 54.6) (end 38.325 53.675) (width 0.5) (layer B.Cu) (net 10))
 (segment (start 38.325 53.675) (end 39 53) (width 0.5) (layer B.Cu) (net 10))
 (segment (start 39 53) (end 46.85 53) (width 0.5) (layer B.Cu) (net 10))
 (segment (start 46.85 53) (end 49.55 50.3) (width 0.5) (layer B.Cu) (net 10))
 (segment (start 49.55 50.3) (end 50.2 50.3) (width 0.5) (layer B.Cu) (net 10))
 (segment (start 50.2 50.3) (end 52.633258 47.866742) (width 0.5) (layer B.Cu) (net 10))
 (segment (start 52.633258 47.866742) (end 52.633258 45.574833) (width 0.5) (layer B.Cu) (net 10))
 (segment (start 52.633258 45.574833) (end 52.424833 45.574833) (width 0.5) (layer B.Cu) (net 10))
 (segment (start 52.424833 45.574833) (end 51.55 44.7) (width 0.5) (layer B.Cu) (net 10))
 (segment (start 51.55 44.7) (end 51.55 42.25) (width 0.5) (layer B.Cu) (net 10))
 (segment (start 51.55 42.25) (end 52.3 41.5) (width 0.5) (layer B.Cu) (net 10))
 (segment (start 52.3 41.5) (end 52.3 38.5) (width 0.5) (layer B.Cu) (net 10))
 (segment (start 52.3 38.5) (end 52.3 38.35) (width 0.5) (layer B.Cu) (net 10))
 (segment (start 52.1 34.1) (end 52.1 32.15) (width 0.5) (layer B.Cu) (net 10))
 (segment (start 52.1 32.15) (end 49.35248 29.40248) (width 0.5) (layer B.Cu) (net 10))
 (segment (start 49.35248 29.40248) (end 48.529242 29.40248) (width 0.5) (layer B.Cu) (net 10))
 (segment (start 36.45 35.955) (end 36.45 39.15) (width 0.5) (layer B.Cu) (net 11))
 (segment (start 34.33 41.27) (end 32.25 41.27) (width 0.5) (layer B.Cu) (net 11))
 (segment (start 36.45 39.15) (end 34.33 41.27) (width 0.5) (layer B.Cu) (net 11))
 (segment (start 28.2 39.9) (end 28.2 40) (width 0.5) (layer B.Cu) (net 12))
 (segment (start 33.125 29.025) (end 28.2 33.95) (width 0.5) (layer B.Cu) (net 12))
 (segment (start 28.2 33.95) (end 28.2 35.05) (width 0.5) (layer B.Cu) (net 12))
 (via (at 28.2 35.05) (size 2.1) (drill 0.8) (layers F.Cu B.Cu) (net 12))
 (segment (start 28.2 35.05) (end 28.2 39.9) (width 0.5) (layer F.Cu) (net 12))
 (via (at 28.2 39.9) (size 2.1) (drill 0.8) (layers F.Cu B.Cu) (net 12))
 (segment (start 34.925 29.025) (end 33.125 29.025) (width 0.5) (layer B.Cu) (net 12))
 (segment (start 30.45 46.35) (end 32.25 46.35) (width 0.5) (layer B.Cu) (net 12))
 (segment (start 30.25 46.15) (end 30.45 46.35) (width 0.5) (layer B.Cu) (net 12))
 (segment (start 30.25 42.05) (end 30.25 46.15) (width 0.5) (layer B.Cu) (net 12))
 (segment (start 28.2 40) (end 30.25 42.05) (width 0.5) (layer B.Cu) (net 12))
 (segment (start 41.85 32.145) (end 41.85 31.15) (width 0.5) (layer B.Cu) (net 12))
 (segment (start 36.2 30.3) (end 34.925 29.025) (width 0.5) (layer B.Cu) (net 12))
 (segment (start 34.925 29.025) (end 34.9 29) (width 0.5) (layer B.Cu) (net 12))
 (segment (start 41 30.3) (end 36.2 30.3) (width 0.5) (layer B.Cu) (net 12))
 (segment (start 41.85 31.15) (end 41 30.3) (width 0.5) (layer B.Cu) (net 12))
 (segment (start 39.4 44.4) (end 43.03 44.4) (width 0.5) (layer B.Cu) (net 13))
 (segment (start 43.03 44.4) (end 43.55 44.92) (width 0.5) (layer B.Cu) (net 13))
 (segment (start 39.4 46.3) (end 39.4 47.675) (width 0.5) (layer B.Cu) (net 14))
 (segment (start 39.4 47.675) (end 38.05 49.025) (width 0.5) (layer B.Cu) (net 14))
 (segment (start 41.85 33.415) (end 43.035 33.415) (width 0.5) (layer B.Cu) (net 15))
 (segment (start 48.7 31.3) (end 46.65 31.3) (width 0.5) (layer B.Cu) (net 15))
 (segment (start 46.65 31.3) (end 46.45 31.1) (width 0.5) (layer B.Cu) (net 15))
 (segment (start 46.45 31.1) (end 45.95 31.1) (width 0.5) (layer B.Cu) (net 15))
 (segment (start 45.95 31.1) (end 45.7 30.85) (width 0.5) (layer B.Cu) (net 15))
 (segment (start 45.7 30.85) (end 44.55 30.85) (width 0.5) (layer B.Cu) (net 15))
 (segment (start 44.55 30.85) (end 43.4 32) (width 0.5) (layer B.Cu) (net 15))
 (segment (start 43.4 32) (end 43.4 33.05) (width 0.5) (layer B.Cu) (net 15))
 (segment (start 43.4 33.05) (end 43.035 33.415) (width 0.5) (layer B.Cu) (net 15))
 (segment (start 48.7 31.3) (end 50.24 32.84) (width 0.5) (layer B.Cu) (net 15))
 (segment (start 50.24 40.46) (end 50.24 38.89) (width 0.5) (layer B.Cu) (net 15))
 (segment (start 49.625 38.275) (end 49.625 36.5) (width 0.5) (layer B.Cu) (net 15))
 (segment (start 50.24 38.89) (end 49.625 38.275) (width 0.5) (layer B.Cu) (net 15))
 (segment (start 50.24 32.84) (end 50.24 33.56) (width 0.5) (layer B.Cu) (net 15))
 (segment (start 50.24 33.56) (end 49.625 34.175) (width 0.5) (layer B.Cu) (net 15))
 (segment (start 49.625 34.175) (end 49.625 36.5) (width 0.5) (layer B.Cu) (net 15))
 (segment (start 49.625 40.245) (end 49.64 40.26) (width 0.5) (layer B.Cu) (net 15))
 (segment (start 49.625 32.655) (end 49.64 32.64) (width 0.5) (layer B.Cu) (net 15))
 (segment (start 46.09 50) (end 46.09 47.335) (width 0.5) (layer B.Cu) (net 16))
 (segment (start 46.09 47.335) (end 46.15 47.275) (width 0.5) (layer B.Cu) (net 16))
 (segment (start 43.785 34.685) (end 45.735 34.685) (width 0.5) (layer B.Cu) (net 17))
 (segment (start 48.05 41.45) (end 49.75 43.15) (width 0.5) (layer B.Cu) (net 17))
 (via (at 49.75 43.15) (size 2.1) (drill 0.8) (layers F.Cu B.Cu) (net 17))
 (segment (start 49.75 43.15) (end 48.6 44.3) (width 0.5) (layer F.Cu) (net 17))
 (segment (start 48.6 44.3) (end 48.6 46.9) (width 0.5) (layer F.Cu) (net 17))
 (via (at 48.6 46.9) (size 2.1) (drill 0.8) (layers F.Cu B.Cu) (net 17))
 (segment (start 48.6 46.9) (end 46.925 45.225) (width 0.5) (layer B.Cu) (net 17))
 (segment (start 46.15 45.225) (end 46.925 45.225) (width 0.5) (layer B.Cu) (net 17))
 (segment (start 43.785 34.685) (end 41.85 34.685) (width 0.5) (layer B.Cu) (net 17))
 (segment (start 47.8 38.7) (end 47.8 41.45) (width 0.5) (layer B.Cu) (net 17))
 (segment (start 47.8 41.45) (end 48.05 41.45) (width 0.5) (layer B.Cu) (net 17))
 (segment (start 47.8 36.75) (end 47.8 38.7) (width 0.5) (layer B.Cu) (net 17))
 (segment (start 45.735 34.685) (end 47.8 36.75) (width 0.5) (layer B.Cu) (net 17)))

